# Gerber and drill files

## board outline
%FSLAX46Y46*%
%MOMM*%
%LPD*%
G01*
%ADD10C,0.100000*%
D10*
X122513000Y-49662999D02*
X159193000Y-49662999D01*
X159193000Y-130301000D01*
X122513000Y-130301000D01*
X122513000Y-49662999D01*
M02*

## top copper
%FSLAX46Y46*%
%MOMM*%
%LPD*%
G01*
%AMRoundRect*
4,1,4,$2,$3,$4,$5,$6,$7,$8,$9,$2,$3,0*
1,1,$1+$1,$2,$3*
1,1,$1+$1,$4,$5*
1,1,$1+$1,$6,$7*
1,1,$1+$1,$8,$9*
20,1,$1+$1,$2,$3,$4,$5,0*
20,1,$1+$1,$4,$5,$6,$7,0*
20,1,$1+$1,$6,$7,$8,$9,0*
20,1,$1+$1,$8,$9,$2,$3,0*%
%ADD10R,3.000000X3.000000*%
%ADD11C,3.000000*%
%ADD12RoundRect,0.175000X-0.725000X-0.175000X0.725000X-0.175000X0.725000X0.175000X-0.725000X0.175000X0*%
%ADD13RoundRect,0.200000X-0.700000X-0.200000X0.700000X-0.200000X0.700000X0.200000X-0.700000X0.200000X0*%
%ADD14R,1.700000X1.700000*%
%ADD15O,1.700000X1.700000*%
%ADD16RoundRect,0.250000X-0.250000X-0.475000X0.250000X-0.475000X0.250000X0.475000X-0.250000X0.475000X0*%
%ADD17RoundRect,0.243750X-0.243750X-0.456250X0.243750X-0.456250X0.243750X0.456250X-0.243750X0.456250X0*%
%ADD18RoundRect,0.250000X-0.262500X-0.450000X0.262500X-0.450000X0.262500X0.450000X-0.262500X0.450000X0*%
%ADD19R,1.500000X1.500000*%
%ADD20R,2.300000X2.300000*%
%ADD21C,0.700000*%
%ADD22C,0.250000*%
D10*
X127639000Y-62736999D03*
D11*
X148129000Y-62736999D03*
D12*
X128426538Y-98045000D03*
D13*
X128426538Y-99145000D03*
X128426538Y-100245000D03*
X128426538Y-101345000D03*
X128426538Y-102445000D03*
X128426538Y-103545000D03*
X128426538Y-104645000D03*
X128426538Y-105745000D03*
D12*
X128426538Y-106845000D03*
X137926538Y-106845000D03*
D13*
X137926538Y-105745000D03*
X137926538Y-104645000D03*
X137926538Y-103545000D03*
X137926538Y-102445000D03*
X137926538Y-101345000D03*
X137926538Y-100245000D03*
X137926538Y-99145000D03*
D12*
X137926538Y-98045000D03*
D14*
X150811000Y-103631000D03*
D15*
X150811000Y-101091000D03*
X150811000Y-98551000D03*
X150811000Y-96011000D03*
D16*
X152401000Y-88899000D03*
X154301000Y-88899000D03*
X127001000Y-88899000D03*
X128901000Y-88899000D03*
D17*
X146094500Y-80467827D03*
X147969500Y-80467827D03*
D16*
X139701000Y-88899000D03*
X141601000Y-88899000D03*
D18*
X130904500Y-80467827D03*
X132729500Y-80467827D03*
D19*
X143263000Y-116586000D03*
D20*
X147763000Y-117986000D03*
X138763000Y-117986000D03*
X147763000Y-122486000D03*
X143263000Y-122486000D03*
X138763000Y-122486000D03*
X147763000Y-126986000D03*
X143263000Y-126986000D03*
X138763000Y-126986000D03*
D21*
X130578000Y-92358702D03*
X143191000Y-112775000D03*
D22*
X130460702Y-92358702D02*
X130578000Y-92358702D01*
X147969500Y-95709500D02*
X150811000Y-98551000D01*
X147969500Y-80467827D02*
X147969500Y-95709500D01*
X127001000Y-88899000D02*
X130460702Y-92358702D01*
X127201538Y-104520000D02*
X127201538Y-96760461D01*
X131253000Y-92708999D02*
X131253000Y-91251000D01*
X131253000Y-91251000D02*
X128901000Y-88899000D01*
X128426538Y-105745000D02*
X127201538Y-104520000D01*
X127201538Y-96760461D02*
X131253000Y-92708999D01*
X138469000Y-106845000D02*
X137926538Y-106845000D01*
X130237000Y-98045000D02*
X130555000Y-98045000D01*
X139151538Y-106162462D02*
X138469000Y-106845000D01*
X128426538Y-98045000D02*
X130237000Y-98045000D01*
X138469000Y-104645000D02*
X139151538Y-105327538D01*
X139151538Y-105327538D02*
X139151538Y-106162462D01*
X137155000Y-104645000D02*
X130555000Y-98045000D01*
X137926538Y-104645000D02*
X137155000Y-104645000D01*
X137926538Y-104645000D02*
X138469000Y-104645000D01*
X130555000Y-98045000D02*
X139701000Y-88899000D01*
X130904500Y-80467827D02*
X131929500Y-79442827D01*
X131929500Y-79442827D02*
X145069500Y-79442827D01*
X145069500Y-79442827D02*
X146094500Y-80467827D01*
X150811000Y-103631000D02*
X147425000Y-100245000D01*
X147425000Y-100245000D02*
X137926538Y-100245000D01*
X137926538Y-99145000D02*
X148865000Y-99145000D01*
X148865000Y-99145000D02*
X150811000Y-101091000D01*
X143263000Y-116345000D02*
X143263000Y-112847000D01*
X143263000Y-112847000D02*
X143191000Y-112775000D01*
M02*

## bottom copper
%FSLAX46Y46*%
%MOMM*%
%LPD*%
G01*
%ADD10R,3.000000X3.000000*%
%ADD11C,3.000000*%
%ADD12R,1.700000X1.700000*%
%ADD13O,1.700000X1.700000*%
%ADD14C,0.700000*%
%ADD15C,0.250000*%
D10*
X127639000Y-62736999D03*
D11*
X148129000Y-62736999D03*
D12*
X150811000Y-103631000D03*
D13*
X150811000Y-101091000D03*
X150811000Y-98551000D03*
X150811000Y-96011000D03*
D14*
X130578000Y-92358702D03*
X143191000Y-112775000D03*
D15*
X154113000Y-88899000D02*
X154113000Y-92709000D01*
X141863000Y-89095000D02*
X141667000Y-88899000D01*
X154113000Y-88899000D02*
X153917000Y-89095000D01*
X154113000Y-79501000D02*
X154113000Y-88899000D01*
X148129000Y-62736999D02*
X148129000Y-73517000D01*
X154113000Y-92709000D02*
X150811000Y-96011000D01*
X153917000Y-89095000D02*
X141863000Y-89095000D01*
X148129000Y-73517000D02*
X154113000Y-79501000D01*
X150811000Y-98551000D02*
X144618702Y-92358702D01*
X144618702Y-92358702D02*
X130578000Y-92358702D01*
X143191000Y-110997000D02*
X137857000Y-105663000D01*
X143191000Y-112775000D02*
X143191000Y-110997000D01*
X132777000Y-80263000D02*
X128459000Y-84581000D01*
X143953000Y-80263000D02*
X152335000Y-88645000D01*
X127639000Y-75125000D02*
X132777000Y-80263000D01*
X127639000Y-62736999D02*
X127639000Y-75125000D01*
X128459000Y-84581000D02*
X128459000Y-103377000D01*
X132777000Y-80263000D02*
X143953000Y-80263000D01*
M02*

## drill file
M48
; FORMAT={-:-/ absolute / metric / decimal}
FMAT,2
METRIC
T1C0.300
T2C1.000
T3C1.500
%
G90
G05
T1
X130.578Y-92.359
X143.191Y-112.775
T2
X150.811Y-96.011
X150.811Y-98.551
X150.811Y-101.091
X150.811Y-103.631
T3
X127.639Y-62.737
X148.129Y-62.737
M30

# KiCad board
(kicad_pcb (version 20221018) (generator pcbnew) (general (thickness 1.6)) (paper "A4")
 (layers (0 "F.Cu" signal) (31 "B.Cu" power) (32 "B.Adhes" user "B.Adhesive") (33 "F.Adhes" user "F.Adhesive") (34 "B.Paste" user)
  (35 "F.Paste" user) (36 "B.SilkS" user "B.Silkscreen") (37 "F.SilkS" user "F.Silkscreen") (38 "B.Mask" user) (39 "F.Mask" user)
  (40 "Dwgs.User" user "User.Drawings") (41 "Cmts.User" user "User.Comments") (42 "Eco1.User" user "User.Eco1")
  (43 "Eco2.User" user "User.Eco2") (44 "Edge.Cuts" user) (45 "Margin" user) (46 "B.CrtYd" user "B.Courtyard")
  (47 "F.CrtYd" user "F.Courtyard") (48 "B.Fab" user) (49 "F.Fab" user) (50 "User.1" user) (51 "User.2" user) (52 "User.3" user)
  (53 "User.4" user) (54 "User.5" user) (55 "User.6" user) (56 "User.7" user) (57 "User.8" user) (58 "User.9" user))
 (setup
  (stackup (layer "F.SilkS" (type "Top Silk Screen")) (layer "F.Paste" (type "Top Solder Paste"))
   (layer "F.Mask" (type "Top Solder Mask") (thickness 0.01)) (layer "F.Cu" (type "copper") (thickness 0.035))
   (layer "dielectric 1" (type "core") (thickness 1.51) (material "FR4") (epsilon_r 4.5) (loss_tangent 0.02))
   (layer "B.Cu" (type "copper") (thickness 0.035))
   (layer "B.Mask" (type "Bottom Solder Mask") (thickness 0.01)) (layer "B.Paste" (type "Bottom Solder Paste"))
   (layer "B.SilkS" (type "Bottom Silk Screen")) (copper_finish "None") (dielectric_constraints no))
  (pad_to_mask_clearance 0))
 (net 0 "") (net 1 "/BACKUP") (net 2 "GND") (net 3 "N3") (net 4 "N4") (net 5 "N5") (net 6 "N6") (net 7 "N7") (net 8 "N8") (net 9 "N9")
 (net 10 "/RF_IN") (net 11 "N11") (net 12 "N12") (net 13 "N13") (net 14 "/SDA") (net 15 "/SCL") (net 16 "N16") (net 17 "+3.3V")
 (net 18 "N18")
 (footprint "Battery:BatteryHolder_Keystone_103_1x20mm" (layer "F.Cu") (at 127.639 62.736999)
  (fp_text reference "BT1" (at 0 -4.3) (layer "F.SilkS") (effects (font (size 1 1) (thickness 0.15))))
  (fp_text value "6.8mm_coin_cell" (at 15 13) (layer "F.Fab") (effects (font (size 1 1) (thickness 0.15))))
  (pad "1" thru_hole rect (at 0 0) (size 3 3) (drill 1.5) (layers "*.Cu" "*.Mask") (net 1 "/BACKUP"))
  (pad "2" thru_hole circle (at 20.49 0) (size 3 3) (drill 1.5) (layers "*.Cu" "*.Mask") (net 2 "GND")))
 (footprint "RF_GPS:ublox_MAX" (layer "F.Cu") (at 133.176538 102.445)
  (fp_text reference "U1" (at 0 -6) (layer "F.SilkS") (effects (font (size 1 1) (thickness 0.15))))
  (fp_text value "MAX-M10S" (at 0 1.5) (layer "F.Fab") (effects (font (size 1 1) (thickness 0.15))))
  (pad "1" smd roundrect (at -4.75 -4.4) (size 1.8 0.7) (layers "F.Cu" "F.Paste" "F.Mask") (roundrect_rratio 0.25) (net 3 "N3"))
  (pad "2" smd roundrect (at -4.75 -3.3) (size 1.8 0.8) (layers "F.Cu" "F.Paste" "F.Mask") (roundrect_rratio 0.25) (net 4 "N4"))
  (pad "3" smd roundrect (at -4.75 -2.2) (size 1.8 0.8) (layers "F.Cu" "F.Paste" "F.Mask") (roundrect_rratio 0.25) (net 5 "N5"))
  (pad "4" smd roundrect (at -4.75 -1.1) (size 1.8 0.8) (layers "F.Cu" "F.Paste" "F.Mask") (roundrect_rratio 0.25) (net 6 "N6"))
  (pad "5" smd roundrect (at -4.75 0) (size 1.8 0.8) (layers "F.Cu" "F.Paste" "F.Mask") (roundrect_rratio 0.25) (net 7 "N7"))
  (pad "6" smd roundrect (at -4.75 1.1) (size 1.8 0.8) (layers "F.Cu" "F.Paste" "F.Mask") (roundrect_rratio 0.25) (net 1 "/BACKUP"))
  (pad "7" smd roundrect (at -4.75 2.2) (size 1.8 0.8) (layers "F.Cu" "F.Paste" "F.Mask") (roundrect_rratio 0.25) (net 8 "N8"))
  (pad "8" smd roundrect (at -4.75 3.3) (size 1.8 0.8) (layers "F.Cu" "F.Paste" "F.Mask") (roundrect_rratio 0.25) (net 8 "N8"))
  (pad "9" smd roundrect (at -4.75 4.4) (size 1.8 0.7) (layers "F.Cu" "F.Paste" "F.Mask") (roundrect_rratio 0.25) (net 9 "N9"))
  (pad "10" smd roundrect (at 4.75 4.4) (size 1.8 0.7) (layers "F.Cu" "F.Paste" "F.Mask") (roundrect_rratio 0.25) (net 3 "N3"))
  (pad "11" smd roundrect (at 4.75 3.3) (size 1.8 0.8) (layers "F.Cu" "F.Paste" "F.Mask") (roundrect_rratio 0.25) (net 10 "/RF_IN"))
  (pad "12" smd roundrect (at 4.75 2.2) (size 1.8 0.8) (layers "F.Cu" "F.Paste" "F.Mask") (roundrect_rratio 0.25) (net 3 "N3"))
  (pad "13" smd roundrect (at 4.75 1.1) (size 1.8 0.8) (layers "F.Cu" "F.Paste" "F.Mask") (roundrect_rratio 0.25) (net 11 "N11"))
  (pad "14" smd roundrect (at 4.75 0) (size 1.8 0.8) (layers "F.Cu" "F.Paste" "F.Mask") (roundrect_rratio 0.25) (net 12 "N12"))
  (pad "15" smd roundrect (at 4.75 -1.1) (size 1.8 0.8) (layers "F.Cu" "F.Paste" "F.Mask") (roundrect_rratio 0.25) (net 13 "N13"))
  (pad "16" smd roundrect (at 4.75 -2.2) (size 1.8 0.8) (layers "F.Cu" "F.Paste" "F.Mask") (roundrect_rratio 0.25) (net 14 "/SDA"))
  (pad "17" smd roundrect (at 4.75 -3.3) (size 1.8 0.8) (layers "F.Cu" "F.Paste" "F.Mask") (roundrect_rratio 0.25) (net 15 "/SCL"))
  (pad "18" smd roundrect (at 4.75 -4.4) (size 1.8 0.7) (layers "F.Cu" "F.Paste" "F.Mask") (roundrect_rratio 0.25) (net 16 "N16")))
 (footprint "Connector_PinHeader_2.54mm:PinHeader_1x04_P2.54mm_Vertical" (layer "F.Cu") (at 150.811 103.631 180)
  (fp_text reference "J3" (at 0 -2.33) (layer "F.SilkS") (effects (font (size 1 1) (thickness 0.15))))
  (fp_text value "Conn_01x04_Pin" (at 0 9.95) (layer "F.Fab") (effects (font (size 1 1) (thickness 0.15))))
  (pad "1" thru_hole rect (at 0 0 180) (size 1.7 1.7) (drill 1) (layers "*.Cu" "*.Mask") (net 14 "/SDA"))
  (pad "2" thru_hole oval (at 0 2.54 180) (size 1.7 1.7) (drill 1) (layers "*.Cu" "*.Mask") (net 15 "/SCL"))
  (pad "3" thru_hole oval (at 0 5.08 180) (size 1.7 1.7) (drill 1) (layers "*.Cu" "*.Mask") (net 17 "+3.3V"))
  (pad "4" thru_hole oval (at 0 7.62 180) (size 1.7 1.7) (drill 1) (layers "*.Cu" "*.Mask") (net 2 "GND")))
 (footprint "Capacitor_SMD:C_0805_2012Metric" (layer "F.Cu") (at 153.351 88.899)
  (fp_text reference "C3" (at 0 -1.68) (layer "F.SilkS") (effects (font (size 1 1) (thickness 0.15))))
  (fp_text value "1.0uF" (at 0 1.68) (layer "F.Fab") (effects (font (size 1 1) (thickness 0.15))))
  (pad "1" smd roundrect (at -0.95 0) (size 1 1.45) (layers "F.Cu" "F.Paste" "F.Mask") (roundrect_rratio 0.25) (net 1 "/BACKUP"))
  (pad "2" smd roundrect (at 0.95 0) (size 1 1.45) (layers "F.Cu" "F.Paste" "F.Mask") (roundrect_rratio 0.25) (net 2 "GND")))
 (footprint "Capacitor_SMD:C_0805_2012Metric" (layer "F.Cu") (at 127.951 88.899)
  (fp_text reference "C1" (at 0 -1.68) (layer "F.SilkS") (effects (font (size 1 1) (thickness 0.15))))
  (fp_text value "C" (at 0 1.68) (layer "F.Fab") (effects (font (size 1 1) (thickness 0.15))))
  (pad "1" smd roundrect (at -0.95 0) (size 1 1.45) (layers "F.Cu" "F.Paste" "F.Mask") (roundrect_rratio 0.25) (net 17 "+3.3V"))
  (pad "2" smd roundrect (at 0.95 0) (size 1 1.45) (layers "F.Cu" "F.Paste" "F.Mask") (roundrect_rratio 0.25) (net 8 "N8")))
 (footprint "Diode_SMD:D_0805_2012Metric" (layer "F.Cu") (at 147.032 80.467827)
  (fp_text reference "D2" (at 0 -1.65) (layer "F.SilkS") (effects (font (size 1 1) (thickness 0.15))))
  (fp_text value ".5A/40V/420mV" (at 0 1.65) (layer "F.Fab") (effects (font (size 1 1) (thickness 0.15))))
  (pad "1" smd roundrect (at -0.9375 0) (size 0.975 1.4) (layers "F.Cu" "F.Paste" "F.Mask") (roundrect_rratio 0.25) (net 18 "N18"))
  (pad "2" smd roundrect (at 0.9375 0) (size 0.975 1.4) (layers "F.Cu" "F.Paste" "F.Mask") (roundrect_rratio 0.25) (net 17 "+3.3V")))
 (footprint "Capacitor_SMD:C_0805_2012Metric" (layer "F.Cu") (at 140.651 88.899)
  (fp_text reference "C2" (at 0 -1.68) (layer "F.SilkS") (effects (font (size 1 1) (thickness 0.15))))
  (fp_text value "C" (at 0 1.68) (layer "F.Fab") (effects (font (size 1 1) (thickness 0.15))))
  (pad "1" smd roundrect (at -0.95 0) (size 1 1.45) (layers "F.Cu" "F.Paste" "F.Mask") (roundrect_rratio 0.25) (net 3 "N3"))
  (pad "2" smd roundrect (at 0.95 0) (size 1 1.45) (layers "F.Cu" "F.Paste" "F.Mask") (roundrect_rratio 0.25) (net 2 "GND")))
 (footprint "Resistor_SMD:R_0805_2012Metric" (layer "F.Cu") (at 131.817 80.467827)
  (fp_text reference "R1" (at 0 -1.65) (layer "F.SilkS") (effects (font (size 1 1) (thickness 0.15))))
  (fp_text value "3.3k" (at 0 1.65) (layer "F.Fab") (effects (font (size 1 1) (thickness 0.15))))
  (pad "1" smd roundrect (at -0.9125 0) (size 1.025 1.4) (layers "F.Cu" "F.Paste" "F.Mask") (roundrect_rratio 0.243902) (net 18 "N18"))
  (pad "2" smd roundrect (at 0.9125 0) (size 1.025 1.4) (layers "F.Cu" "F.Paste" "F.Mask") (roundrect_rratio 0.243902) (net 1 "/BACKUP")))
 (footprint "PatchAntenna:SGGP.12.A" (layer "F.Cu") (at 142.755 124.062 180)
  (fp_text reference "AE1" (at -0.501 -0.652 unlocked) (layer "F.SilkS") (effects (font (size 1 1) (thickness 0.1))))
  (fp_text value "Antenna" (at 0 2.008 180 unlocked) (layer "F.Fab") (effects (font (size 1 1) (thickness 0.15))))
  (pad "1" smd rect (at -0.508 7.476 180) (size 1.5 1.5) (layers "F.Cu" "F.Paste" "F.Mask") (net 10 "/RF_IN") (thermal_bridge_angle 45))
  (pad "2" smd rect (at -5.008 6.076 180) (size 2.3 2.3) (layers "F.Cu" "F.Paste" "F.Mask") (thermal_bridge_angle 45))
  (pad "3" smd rect (at 3.992 6.076 180) (size 2.3 2.3) (layers "F.Cu" "F.Paste" "F.Mask") (thermal_bridge_angle 45))
  (pad "4" smd rect (at -5.008 1.576 180) (size 2.3 2.3) (layers "F.Cu" "F.Paste" "F.Mask") (thermal_bridge_angle 45))
  (pad "5" smd rect (at -0.508 1.576 180) (size 2.3 2.3) (layers "F.Cu" "F.Paste" "F.Mask") (thermal_bridge_angle 45))
  (pad "6" smd rect (at 3.992 1.576 180) (size 2.3 2.3) (layers "F.Cu" "F.Paste" "F.Mask") (thermal_bridge_angle 45))
  (pad "7" smd rect (at -5.008 -2.924 180) (size 2.3 2.3) (layers "F.Cu" "F.Paste" "F.Mask") (thermal_bridge_angle 45))
  (pad "8" smd rect (at -0.508 -2.924 180) (size 2.3 2.3) (layers "F.Cu" "F.Paste" "F.Mask") (thermal_bridge_angle 45))
  (pad "9" smd rect (at 3.992 -2.924 180) (size 2.3 2.3) (layers "F.Cu" "F.Paste" "F.Mask") (thermal_bridge_angle 45)))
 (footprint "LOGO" (layer "F.Cu") (at 127.443 53.847)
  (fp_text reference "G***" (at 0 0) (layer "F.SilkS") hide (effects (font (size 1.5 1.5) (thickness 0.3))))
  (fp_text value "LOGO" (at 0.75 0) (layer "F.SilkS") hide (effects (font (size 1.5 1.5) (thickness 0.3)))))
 (gr_rect (start 122.513 49.662999) (end 159.193 130.301) (stroke (width 0.1) (type default)) (fill none) (layer "Edge.Cuts"))
 (segment (start 154.113 88.899) (end 154.113 92.709) (width 0.25) (layer "B.Cu") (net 2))
 (segment (start 141.863 89.095) (end 141.667 88.899) (width 0.25) (layer "B.Cu") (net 2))
 (segment (start 154.113 88.899) (end 153.917 89.095) (width 0.25) (layer "B.Cu") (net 2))
 (segment (start 154.113 79.501) (end 154.113 88.899) (width 0.25) (layer "B.Cu") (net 2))
 (segment (start 148.129 62.736999) (end 148.129 73.517) (width 0.25) (layer "B.Cu") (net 2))
 (segment (start 154.113 92.709) (end 150.811 96.011) (width 0.25) (layer "B.Cu") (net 2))
 (segment (start 153.917 89.095) (end 141.863 89.095) (width 0.25) (layer "B.Cu") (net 2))
 (segment (start 148.129 73.517) (end 154.113 79.501) (width 0.25) (layer "B.Cu") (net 2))
 (segment (start 130.460702 92.358702) (end 130.578 92.358702) (width 0.25) (layer "F.Cu") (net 17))
 (segment (start 147.9695 95.7095) (end 150.811 98.551) (width 0.25) (layer "F.Cu") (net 17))
 (segment (start 147.9695 80.467827) (end 147.9695 95.7095) (width 0.25) (layer "F.Cu") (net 17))
 (segment (start 127.001 88.899) (end 130.460702 92.358702) (width 0.25) (layer "F.Cu") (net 17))
 (via (at 130.578 92.358702) (size 0.7) (drill 0.3) (layers "F.Cu" "B.Cu") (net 17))
 (segment (start 150.811 98.551) (end 144.618702 92.358702) (width 0.25) (layer "B.Cu") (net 17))
 (segment (start 144.618702 92.358702) (end 130.578 92.358702) (width 0.25) (layer "B.Cu") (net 17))
 (segment (start 127.201538 104.52) (end 127.201538 96.760461) (width 0.25) (layer "F.Cu") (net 8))
 (segment (start 131.253 92.708999) (end 131.253 91.251) (width 0.25) (layer "F.Cu") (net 8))
 (segment (start 131.253 91.251) (end 128.901 88.899) (width 0.25) (layer "F.Cu") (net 8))
 (segment (start 128.426538 105.745) (end 127.201538 104.52) (width 0.25) (layer "F.Cu") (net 8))
 (segment (start 127.201538 96.760461) (end 131.253 92.708999) (width 0.25) (layer "F.Cu") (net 8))
 (segment (start 138.469 106.845) (end 137.926538 106.845) (width 0.25) (layer "F.Cu") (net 3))
 (segment (start 130.237 98.045) (end 130.555 98.045) (width 0.25) (layer "F.Cu") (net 3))
 (segment (start 139.151538 106.162462) (end 138.469 106.845) (width 0.25) (layer "F.Cu") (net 3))
 (segment (start 128.426538 98.045) (end 130.237 98.045) (width 0.25) (layer "F.Cu") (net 3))
 (segment (start 138.469 104.645) (end 139.151538 105.327538) (width 0.25) (layer "F.Cu") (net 3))
 (segment (start 139.151538 105.327538) (end 139.151538 106.162462) (width 0.25) (layer "F.Cu") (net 3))
 (segment (start 137.155 104.645) (end 130.555 98.045) (width 0.25) (layer "F.Cu") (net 3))
 (segment (start 137.926538 104.645) (end 137.155 104.645) (width 0.25) (layer "F.Cu") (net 3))
 (segment (start 137.926538 104.645) (end 138.469 104.645) (width 0.25) (layer "F.Cu") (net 3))
 (segment (start 130.555 98.045) (end 139.701 88.899) (width 0.25) (layer "F.Cu") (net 3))
 (segment (start 130.9045 80.467827) (end 131.9295 79.442827) (width 0.25) (layer "F.Cu") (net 18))
 (segment (start 131.9295 79.442827) (end 145.0695 79.442827) (width 0.25) (layer "F.Cu") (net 18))
 (segment (start 145.0695 79.442827) (end 146.0945 80.467827) (width 0.25) (layer "F.Cu") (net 18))
 (segment (start 150.811 103.631) (end 147.425 100.245) (width 0.25) (layer "F.Cu") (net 14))
 (segment (start 147.425 100.245) (end 137.926538 100.245) (width 0.25) (layer "F.Cu") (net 14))
 (segment (start 137.926538 99.145) (end 148.865 99.145) (width 0.25) (layer "F.Cu") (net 15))
 (segment (start 148.865 99.145) (end 150.811 101.091) (width 0.25) (layer "F.Cu") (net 15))
 (segment (start 143.263 116.345) (end 143.263 112.847) (width 0.25) (layer "F.Cu") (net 10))
 (segment (start 143.263 112.847) (end 143.191 112.775) (width 0.25) (layer "F.Cu") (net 10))
 (via (at 143.191 112.775) (size 0.7) (drill 0.3) (layers "F.Cu" "B.Cu") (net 10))
 (segment (start 143.191 110.997) (end 137.857 105.663) (width 0.25) (layer "B.Cu") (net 10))
 (segment (start 143.191 112.775) (end 143.191 110.997) (width 0.25) (layer "B.Cu") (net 10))
 (segment (start 132.777 80.263) (end 128.459 84.581) (width 0.25) (layer "B.Cu") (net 1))
 (segment (start 143.953 80.263) (end 152.335 88.645) (width 0.25) (layer "B.Cu") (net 1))
 (segment (start 127.639 75.125) (end 132.777 80.263) (width 0.25) (layer "B.Cu") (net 1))
 (segment (start 127.639 62.736999) (end 127.639 75.125) (width 0.25) (layer "B.Cu") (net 1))
 (segment (start 128.459 84.581) (end 128.459 103.377) (width 0.25) (layer "B.Cu") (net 1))
 (segment (start 132.777 80.263) (end 143.953 80.263) (width 0.25) (layer "B.Cu") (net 1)))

